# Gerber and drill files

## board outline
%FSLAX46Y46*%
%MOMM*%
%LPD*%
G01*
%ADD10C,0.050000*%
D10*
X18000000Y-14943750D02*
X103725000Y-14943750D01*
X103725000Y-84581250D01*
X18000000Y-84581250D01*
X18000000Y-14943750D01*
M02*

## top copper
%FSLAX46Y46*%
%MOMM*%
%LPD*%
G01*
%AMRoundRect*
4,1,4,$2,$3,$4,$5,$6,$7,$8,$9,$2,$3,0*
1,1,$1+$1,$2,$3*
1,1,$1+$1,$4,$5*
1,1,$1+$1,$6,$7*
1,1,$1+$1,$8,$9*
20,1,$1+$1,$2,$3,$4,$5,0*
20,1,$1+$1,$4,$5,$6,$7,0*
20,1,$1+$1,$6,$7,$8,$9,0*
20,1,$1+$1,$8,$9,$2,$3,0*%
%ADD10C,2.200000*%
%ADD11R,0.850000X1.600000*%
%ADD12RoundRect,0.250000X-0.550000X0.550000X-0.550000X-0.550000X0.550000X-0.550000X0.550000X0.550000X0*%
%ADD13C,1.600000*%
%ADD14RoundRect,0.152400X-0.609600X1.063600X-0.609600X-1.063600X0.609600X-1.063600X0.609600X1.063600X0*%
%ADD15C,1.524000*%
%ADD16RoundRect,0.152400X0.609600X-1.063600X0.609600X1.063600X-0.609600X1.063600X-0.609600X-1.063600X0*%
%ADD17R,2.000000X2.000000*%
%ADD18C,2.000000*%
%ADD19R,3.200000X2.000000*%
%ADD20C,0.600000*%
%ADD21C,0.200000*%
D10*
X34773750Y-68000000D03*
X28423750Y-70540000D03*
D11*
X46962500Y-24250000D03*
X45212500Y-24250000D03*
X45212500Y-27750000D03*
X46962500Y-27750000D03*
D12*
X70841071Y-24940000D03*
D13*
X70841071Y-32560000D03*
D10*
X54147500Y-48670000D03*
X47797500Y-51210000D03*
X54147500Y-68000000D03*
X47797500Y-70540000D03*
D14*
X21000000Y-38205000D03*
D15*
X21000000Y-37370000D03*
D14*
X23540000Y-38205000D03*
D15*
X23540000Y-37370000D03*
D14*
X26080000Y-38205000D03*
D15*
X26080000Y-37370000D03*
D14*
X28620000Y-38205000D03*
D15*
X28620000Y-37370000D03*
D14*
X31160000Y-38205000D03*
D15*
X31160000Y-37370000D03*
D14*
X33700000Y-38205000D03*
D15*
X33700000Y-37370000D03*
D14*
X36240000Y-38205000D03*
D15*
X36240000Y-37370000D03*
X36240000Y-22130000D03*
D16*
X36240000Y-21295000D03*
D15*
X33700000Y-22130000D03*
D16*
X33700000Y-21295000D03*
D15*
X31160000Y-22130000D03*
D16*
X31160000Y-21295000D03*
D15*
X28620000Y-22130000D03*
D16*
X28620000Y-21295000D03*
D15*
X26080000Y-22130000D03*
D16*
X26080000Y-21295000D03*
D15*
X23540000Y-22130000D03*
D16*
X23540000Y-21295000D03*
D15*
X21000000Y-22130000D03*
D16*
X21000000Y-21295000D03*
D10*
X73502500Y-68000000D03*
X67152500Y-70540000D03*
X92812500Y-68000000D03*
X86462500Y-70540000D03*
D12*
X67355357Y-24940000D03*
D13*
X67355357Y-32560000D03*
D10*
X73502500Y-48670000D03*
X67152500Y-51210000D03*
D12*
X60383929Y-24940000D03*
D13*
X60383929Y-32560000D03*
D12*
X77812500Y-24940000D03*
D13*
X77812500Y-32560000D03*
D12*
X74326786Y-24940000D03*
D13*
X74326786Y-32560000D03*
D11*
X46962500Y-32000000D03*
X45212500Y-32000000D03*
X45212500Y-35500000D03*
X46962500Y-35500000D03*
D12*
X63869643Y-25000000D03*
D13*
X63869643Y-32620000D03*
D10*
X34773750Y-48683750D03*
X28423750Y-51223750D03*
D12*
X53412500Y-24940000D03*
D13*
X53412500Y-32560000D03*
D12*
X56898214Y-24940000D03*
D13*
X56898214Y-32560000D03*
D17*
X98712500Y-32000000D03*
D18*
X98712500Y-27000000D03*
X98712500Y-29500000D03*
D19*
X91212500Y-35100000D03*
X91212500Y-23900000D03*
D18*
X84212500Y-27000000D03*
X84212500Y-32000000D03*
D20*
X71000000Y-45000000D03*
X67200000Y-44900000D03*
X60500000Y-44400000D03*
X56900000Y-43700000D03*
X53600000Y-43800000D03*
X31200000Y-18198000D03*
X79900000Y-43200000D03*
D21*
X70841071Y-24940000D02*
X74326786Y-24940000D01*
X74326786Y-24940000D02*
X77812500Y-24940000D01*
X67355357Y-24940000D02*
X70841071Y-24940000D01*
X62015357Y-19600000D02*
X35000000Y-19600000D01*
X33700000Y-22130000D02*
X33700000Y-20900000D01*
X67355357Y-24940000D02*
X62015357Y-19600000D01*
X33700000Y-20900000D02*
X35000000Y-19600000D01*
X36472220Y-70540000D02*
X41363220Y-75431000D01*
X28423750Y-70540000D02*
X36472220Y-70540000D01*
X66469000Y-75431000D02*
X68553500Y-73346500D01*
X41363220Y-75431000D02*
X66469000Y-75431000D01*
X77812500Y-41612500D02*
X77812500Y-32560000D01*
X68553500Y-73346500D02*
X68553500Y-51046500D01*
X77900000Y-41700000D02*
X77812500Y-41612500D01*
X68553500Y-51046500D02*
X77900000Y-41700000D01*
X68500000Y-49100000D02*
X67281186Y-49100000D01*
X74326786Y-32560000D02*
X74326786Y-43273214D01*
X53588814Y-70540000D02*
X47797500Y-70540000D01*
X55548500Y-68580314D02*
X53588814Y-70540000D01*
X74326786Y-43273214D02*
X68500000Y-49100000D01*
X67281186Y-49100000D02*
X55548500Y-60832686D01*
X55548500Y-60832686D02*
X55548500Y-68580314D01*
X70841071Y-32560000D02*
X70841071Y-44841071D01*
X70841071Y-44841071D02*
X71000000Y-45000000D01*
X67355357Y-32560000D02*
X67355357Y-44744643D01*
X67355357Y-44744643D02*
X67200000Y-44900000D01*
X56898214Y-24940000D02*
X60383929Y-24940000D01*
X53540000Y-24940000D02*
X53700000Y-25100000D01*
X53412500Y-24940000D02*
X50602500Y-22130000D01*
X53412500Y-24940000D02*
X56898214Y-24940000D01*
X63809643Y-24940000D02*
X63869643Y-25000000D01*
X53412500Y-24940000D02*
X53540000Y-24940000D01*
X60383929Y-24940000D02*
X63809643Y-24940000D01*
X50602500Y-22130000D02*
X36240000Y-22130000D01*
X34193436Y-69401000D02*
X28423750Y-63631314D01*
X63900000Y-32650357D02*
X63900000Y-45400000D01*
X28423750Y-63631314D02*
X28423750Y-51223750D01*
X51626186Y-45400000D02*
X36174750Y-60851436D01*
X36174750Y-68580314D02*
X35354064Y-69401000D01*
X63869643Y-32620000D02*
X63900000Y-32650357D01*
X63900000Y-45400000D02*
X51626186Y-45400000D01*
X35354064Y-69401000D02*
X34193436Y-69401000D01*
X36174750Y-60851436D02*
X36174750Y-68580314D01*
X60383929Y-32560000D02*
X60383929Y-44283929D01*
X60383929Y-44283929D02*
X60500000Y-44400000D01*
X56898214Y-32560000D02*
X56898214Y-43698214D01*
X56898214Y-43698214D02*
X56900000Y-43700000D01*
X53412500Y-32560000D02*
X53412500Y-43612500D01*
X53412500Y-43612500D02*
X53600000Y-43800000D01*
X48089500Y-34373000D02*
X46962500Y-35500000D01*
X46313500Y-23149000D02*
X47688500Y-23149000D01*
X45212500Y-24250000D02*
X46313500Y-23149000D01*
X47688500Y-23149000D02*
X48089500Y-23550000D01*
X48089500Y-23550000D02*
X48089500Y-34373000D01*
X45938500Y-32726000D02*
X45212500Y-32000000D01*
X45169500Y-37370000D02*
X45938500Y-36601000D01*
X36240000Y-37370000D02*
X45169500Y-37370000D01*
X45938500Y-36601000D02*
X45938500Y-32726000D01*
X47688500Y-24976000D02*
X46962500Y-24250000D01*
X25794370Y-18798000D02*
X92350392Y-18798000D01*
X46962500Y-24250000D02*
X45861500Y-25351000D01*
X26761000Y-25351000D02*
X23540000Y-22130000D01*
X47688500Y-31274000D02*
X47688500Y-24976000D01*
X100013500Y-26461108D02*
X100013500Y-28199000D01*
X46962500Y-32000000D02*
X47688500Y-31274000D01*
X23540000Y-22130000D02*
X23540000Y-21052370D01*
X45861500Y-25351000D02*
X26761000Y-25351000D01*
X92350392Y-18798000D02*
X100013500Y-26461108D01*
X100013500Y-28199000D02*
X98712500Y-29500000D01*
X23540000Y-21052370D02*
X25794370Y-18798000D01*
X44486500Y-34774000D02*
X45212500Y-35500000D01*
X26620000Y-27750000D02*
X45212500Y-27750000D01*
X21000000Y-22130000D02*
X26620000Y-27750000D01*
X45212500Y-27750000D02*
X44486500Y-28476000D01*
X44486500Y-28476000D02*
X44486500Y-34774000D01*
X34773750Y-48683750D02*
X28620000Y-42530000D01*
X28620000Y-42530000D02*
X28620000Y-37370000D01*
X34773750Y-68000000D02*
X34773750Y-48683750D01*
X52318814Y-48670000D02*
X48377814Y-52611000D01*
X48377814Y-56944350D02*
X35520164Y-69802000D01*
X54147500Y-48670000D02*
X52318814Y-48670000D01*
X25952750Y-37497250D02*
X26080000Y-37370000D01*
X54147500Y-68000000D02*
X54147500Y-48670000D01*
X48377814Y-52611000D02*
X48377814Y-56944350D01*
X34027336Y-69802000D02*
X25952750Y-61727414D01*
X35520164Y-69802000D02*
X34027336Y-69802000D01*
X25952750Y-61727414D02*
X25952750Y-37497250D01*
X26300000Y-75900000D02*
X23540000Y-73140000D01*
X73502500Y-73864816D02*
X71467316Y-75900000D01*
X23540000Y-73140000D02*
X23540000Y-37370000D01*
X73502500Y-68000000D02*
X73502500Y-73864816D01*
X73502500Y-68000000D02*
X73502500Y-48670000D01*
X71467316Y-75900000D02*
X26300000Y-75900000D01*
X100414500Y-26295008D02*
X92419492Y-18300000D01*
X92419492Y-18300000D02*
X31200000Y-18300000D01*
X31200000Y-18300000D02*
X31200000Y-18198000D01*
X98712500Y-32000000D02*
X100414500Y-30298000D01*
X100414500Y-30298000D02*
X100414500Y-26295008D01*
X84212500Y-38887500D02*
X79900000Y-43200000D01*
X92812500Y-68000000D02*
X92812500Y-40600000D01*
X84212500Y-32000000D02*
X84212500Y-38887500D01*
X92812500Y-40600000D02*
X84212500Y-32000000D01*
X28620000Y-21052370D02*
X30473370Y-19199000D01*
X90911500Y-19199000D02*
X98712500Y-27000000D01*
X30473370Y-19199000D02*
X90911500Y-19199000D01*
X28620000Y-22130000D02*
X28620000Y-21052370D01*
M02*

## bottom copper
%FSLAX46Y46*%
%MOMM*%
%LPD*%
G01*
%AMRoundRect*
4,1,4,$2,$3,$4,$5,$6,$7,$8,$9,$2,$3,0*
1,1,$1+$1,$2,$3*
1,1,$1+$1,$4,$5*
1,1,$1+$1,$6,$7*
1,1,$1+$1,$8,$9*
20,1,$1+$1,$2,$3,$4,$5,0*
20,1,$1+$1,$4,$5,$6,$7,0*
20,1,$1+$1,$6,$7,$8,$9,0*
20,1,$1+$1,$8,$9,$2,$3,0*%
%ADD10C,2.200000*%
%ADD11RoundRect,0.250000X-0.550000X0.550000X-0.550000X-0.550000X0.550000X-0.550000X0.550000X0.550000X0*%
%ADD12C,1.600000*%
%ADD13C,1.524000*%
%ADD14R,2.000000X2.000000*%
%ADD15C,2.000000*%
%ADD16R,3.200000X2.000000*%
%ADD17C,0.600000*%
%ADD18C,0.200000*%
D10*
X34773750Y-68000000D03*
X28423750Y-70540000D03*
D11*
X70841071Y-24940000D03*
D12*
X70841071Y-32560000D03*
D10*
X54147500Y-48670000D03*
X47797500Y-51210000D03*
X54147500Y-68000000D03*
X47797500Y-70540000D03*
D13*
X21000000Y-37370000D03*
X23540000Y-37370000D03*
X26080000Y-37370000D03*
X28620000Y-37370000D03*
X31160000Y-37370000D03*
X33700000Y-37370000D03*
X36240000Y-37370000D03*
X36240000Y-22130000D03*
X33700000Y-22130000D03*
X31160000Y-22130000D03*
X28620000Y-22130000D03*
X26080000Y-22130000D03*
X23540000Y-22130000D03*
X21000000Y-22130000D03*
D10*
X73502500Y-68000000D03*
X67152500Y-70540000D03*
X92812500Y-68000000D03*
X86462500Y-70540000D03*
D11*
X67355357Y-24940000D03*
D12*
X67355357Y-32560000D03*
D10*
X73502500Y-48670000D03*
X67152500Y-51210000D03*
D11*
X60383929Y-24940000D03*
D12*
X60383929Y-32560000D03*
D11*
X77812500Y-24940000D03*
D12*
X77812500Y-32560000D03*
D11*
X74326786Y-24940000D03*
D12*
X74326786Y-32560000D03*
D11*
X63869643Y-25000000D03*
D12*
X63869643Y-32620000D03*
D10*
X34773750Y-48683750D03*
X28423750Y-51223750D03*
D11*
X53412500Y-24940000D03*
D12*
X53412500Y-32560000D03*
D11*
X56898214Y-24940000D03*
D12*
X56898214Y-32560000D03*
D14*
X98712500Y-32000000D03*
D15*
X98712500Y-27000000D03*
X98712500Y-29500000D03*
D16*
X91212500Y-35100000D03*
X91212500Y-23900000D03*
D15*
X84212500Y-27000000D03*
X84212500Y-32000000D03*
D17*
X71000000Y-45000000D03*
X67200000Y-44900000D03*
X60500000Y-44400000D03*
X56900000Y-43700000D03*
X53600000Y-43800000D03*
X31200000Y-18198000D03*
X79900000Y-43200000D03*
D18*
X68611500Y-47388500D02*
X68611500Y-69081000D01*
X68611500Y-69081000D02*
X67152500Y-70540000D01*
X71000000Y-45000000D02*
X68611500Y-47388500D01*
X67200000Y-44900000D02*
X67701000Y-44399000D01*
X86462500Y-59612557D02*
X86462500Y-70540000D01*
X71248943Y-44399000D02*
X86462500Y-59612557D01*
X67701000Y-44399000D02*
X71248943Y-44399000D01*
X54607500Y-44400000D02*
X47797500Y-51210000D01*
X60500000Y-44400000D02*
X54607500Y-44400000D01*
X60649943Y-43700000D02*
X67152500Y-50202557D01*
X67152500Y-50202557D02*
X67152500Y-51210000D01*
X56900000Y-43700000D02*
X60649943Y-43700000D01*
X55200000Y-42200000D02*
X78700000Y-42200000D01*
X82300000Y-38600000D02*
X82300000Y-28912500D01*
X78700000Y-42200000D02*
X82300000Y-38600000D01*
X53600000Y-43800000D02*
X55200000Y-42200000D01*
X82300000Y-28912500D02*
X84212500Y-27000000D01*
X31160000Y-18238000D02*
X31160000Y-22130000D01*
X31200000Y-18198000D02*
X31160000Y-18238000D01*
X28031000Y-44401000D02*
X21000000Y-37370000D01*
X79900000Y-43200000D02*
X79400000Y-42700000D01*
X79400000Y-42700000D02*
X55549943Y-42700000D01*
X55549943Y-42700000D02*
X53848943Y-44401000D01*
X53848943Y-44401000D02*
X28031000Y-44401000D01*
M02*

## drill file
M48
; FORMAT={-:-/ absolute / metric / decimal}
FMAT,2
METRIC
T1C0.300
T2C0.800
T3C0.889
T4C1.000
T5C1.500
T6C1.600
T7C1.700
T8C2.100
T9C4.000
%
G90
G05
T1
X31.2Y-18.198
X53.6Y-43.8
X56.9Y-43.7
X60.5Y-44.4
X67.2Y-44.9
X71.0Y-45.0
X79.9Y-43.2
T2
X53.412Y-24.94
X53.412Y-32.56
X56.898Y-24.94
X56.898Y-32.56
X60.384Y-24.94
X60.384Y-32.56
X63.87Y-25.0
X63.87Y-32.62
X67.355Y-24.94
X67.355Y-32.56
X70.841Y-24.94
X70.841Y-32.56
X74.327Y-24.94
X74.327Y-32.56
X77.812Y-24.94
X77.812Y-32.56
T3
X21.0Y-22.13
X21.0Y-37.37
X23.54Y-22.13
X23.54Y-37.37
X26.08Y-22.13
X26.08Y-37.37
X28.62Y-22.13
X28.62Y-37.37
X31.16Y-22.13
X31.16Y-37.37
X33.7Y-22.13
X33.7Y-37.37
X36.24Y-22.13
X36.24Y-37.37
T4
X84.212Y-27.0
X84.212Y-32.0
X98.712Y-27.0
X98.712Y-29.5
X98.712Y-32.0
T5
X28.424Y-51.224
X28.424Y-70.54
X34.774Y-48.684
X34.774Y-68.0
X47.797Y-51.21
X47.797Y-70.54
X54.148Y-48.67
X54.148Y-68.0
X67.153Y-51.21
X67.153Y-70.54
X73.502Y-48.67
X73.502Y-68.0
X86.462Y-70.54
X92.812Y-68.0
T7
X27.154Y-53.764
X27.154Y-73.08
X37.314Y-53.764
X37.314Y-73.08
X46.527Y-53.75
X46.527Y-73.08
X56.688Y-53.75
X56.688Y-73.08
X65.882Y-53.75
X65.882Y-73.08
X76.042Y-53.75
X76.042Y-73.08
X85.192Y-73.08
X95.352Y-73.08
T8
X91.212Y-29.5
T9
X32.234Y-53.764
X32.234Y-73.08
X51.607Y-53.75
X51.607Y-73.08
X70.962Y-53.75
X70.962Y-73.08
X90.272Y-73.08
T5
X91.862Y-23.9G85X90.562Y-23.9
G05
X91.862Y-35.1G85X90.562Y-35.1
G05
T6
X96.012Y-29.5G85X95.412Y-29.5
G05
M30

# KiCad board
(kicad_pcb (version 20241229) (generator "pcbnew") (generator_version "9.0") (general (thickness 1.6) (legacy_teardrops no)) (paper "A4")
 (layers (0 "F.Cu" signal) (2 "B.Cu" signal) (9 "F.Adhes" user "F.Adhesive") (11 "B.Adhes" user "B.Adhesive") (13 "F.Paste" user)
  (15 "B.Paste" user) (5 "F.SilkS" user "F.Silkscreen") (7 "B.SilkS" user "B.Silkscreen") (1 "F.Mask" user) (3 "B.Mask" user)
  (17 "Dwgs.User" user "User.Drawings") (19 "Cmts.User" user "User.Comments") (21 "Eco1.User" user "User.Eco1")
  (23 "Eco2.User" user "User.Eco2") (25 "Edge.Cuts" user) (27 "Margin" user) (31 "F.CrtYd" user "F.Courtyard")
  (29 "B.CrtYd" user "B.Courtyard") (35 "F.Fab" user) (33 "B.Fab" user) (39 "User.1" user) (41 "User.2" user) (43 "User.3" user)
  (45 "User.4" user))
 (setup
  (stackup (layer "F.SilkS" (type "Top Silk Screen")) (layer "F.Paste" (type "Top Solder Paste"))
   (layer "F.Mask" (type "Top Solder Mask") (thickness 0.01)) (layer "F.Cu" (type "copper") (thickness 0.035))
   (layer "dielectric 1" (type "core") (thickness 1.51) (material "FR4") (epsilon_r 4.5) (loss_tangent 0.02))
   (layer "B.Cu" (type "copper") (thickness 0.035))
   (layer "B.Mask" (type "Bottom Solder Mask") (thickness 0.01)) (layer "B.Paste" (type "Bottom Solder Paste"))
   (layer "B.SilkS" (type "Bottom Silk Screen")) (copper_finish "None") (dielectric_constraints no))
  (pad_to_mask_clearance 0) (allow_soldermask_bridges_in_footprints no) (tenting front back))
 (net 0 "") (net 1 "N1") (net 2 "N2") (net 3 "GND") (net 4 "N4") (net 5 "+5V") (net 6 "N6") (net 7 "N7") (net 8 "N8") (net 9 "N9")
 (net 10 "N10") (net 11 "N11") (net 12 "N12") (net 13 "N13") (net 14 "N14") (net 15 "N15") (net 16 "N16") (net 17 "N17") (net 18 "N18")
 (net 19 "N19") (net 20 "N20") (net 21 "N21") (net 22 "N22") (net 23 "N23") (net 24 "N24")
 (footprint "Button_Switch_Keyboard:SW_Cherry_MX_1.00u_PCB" (layer "F.Cu") (at 34.77375 68)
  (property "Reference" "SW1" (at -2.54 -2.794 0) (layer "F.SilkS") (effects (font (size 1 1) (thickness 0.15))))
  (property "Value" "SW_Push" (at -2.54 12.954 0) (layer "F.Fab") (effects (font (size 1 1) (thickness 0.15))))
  (pad "" np_thru_hole circle (at -7.62 5.08) (size 1.7 1.7) (drill 1.7) (layers "*.Cu" "*.Mask"))
  (pad "" np_thru_hole circle (at -2.54 5.08) (size 4 4) (drill 4) (layers "*.Cu" "*.Mask"))
  (pad "" np_thru_hole circle (at 2.54 5.08) (size 1.7 1.7) (drill 1.7) (layers "*.Cu" "*.Mask"))
  (pad "1" thru_hole circle (at 0 0) (size 2.2 2.2) (drill 1.5) (layers "*.Cu" "*.Mask") (remove_unused_layers no) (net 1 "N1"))
  (pad "2" thru_hole circle (at -6.35 2.54) (size 2.2 2.2) (drill 1.5) (layers "*.Cu" "*.Mask") (remove_unused_layers no) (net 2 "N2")))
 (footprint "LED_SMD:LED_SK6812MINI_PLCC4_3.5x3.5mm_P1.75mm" (layer "F.Cu") (at 46.0875 26 -90)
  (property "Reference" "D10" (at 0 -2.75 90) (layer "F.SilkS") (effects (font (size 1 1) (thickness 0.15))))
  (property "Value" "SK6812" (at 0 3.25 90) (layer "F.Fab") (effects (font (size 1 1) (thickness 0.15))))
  (pad "1" smd rect (at -1.75 -0.875 270) (size 1.6 0.85) (layers "F.Cu" "F.Mask" "F.Paste") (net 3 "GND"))
  (pad "2" smd rect (at -1.75 0.875 270) (size 1.6 0.85) (layers "F.Cu" "F.Mask" "F.Paste") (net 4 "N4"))
  (pad "3" smd rect (at 1.75 0.875 270) (size 1.6 0.85) (layers "F.Cu" "F.Mask" "F.Paste") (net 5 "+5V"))
  (pad "4" smd rect (at 1.75 -0.875 270) (size 1.6 0.85) (layers "F.Cu" "F.Mask" "F.Paste") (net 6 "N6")))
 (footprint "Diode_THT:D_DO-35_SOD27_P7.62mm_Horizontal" (layer "F.Cu") (at 70.841071 24.94 -90)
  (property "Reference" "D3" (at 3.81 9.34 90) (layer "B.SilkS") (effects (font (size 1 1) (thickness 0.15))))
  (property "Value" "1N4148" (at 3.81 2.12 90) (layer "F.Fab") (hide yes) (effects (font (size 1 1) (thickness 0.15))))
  (pad "1" thru_hole roundrect (at 0 0 270) (size 1.6 1.6) (drill 0.8) (layers "*.Cu" "*.Mask") (remove_unused_layers no)
   (roundrect_rratio 0.15625) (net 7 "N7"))
  (pad "2" thru_hole circle (at 7.62 0 270) (size 1.6 1.6) (drill 0.8) (layers "*.Cu" "*.Mask") (remove_unused_layers no) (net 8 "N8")))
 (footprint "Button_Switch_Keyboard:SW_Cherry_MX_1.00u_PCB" (layer "F.Cu") (at 54.1475 48.67)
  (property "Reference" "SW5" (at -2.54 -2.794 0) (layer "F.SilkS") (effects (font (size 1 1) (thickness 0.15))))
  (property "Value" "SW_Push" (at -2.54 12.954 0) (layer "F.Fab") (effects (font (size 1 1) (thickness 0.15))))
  (pad "" np_thru_hole circle (at -7.62 5.08) (size 1.7 1.7) (drill 1.7) (layers "*.Cu" "*.Mask"))
  (pad "" np_thru_hole circle (at -2.54 5.08) (size 4 4) (drill 4) (layers "*.Cu" "*.Mask"))
  (pad "" np_thru_hole circle (at 2.54 5.08) (size 1.7 1.7) (drill 1.7) (layers "*.Cu" "*.Mask"))
  (pad "1" thru_hole circle (at 0 0) (size 2.2 2.2) (drill 1.5) (layers "*.Cu" "*.Mask") (remove_unused_layers no) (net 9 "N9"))
  (pad "2" thru_hole circle (at -6.35 2.54) (size 2.2 2.2) (drill 1.5) (layers "*.Cu" "*.Mask") (remove_unused_layers no) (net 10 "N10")))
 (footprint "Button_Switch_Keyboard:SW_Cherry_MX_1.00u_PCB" (layer "F.Cu") (at 54.1475 68)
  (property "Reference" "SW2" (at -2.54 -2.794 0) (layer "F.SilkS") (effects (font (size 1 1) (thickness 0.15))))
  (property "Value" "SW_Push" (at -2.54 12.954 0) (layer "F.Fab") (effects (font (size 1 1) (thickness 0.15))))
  (pad "" np_thru_hole circle (at -7.62 5.08) (size 1.7 1.7) (drill 1.7) (layers "*.Cu" "*.Mask"))
  (pad "" np_thru_hole circle (at -2.54 5.08) (size 4 4) (drill 4) (layers "*.Cu" "*.Mask"))
  (pad "" np_thru_hole circle (at 2.54 5.08) (size 1.7 1.7) (drill 1.7) (layers "*.Cu" "*.Mask"))
  (pad "1" thru_hole circle (at 0 0) (size 2.2 2.2) (drill 1.5) (layers "*.Cu" "*.Mask") (remove_unused_layers no) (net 9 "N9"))
  (pad "2" thru_hole circle (at -6.35 2.54) (size 2.2 2.2) (drill 1.5) (layers "*.Cu" "*.Mask") (remove_unused_layers no) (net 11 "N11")))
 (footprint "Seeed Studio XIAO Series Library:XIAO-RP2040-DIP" (layer "F.Cu") (at 28.62 29.75 90)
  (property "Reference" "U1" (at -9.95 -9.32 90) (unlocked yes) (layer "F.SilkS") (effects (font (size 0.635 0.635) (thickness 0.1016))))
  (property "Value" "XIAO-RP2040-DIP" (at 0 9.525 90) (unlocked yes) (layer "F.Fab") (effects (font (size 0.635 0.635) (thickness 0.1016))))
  (pad "1" smd roundrect (at -8.455 -7.62 270) (size 2.432 1.524) (layers "F.Cu" "F.Mask") (roundrect_rratio 0.1) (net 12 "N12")
   (thermal_bridge_angle 45))
  (pad "1" thru_hole circle (at -7.62 -7.62 270) (size 1.524 1.524) (drill 0.889) (layers "*.Cu" "*.Mask") (remove_unused_layers no)
   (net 12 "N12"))
  (pad "2" smd roundrect (at -8.455 -5.08 270) (size 2.432 1.524) (layers "F.Cu" "F.Mask") (roundrect_rratio 0.1) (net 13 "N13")
   (thermal_bridge_angle 45))
  (pad "2" thru_hole circle (at -7.62 -5.08 270) (size 1.524 1.524) (drill 0.889) (layers "*.Cu" "*.Mask") (remove_unused_layers no)
   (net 13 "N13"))
  (pad "3" smd roundrect (at -8.455 -2.54 270) (size 2.432 1.524) (layers "F.Cu" "F.Mask") (roundrect_rratio 0.1) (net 9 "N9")
   (thermal_bridge_angle 45))
  (pad "3" thru_hole circle (at -7.62 -2.54 270) (size 1.524 1.524) (drill 0.889) (layers "*.Cu" "*.Mask") (remove_unused_layers no)
   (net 9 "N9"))
  (pad "4" smd roundrect (at -8.455 0 270) (size 2.432 1.524) (layers "F.Cu" "F.Mask") (roundrect_rratio 0.1) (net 1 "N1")
   (thermal_bridge_angle 45))
  (pad "4" thru_hole circle (at -7.62 0 270) (size 1.524 1.524) (drill 0.889) (layers "*.Cu" "*.Mask") (remove_unused_layers no)
   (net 1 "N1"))
  (pad "5" smd roundrect (at -8.455 2.54 270) (size 2.432 1.524) (layers "F.Cu" "F.Mask") (roundrect_rratio 0.1) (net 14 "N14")
   (thermal_bridge_angle 45))
  (pad "5" thru_hole circle (at -7.62 2.54 270) (size 1.524 1.524) (drill 0.889) (layers "*.Cu" "*.Mask") (remove_unused_layers no)
   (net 14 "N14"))
  (pad "6" smd roundrect (at -8.455 5.08 270) (size 2.432 1.524) (layers "F.Cu" "F.Mask") (roundrect_rratio 0.1) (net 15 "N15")
   (thermal_bridge_angle 45))
  (pad "6" thru_hole circle (at -7.62 5.08 270) (size 1.524 1.524) (drill 0.889) (layers "*.Cu" "*.Mask") (remove_unused_layers no)
   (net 15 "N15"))
  (pad "7" smd roundrect (at -8.455 7.62 270) (size 2.432 1.524) (layers "F.Cu" "F.Mask") (roundrect_rratio 0.1) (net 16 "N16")
   (thermal_bridge_angle 45))
  (pad "7" thru_hole circle (at -7.62 7.62 270) (size 1.524 1.524) (drill 0.889) (layers "*.Cu" "*.Mask") (remove_unused_layers no)
   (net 16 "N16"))
  (pad "8" thru_hole circle (at 7.62 7.62 90) (size 1.524 1.524) (drill 0.889) (layers "*.Cu" "*.Mask") (remove_unused_layers no)
   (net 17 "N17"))
  (pad "8" smd roundrect (at 8.455 7.62 90) (size 2.432 1.524) (layers "F.Cu" "F.Mask") (roundrect_rratio 0.1) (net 17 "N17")
   (thermal_bridge_angle 45))
  (pad "9" thru_hole circle (at 7.62 5.08 90) (size 1.524 1.524) (drill 0.889) (layers "*.Cu" "*.Mask") (remove_unused_layers no)
   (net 7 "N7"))
  (pad "9" smd roundrect (at 8.455 5.08 90) (size 2.432 1.524) (layers "F.Cu" "F.Mask") (roundrect_rratio 0.1) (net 7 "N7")
   (thermal_bridge_angle 45))
  (pad "10" thru_hole circle (at 7.62 2.54 90) (size 1.524 1.524) (drill 0.889) (layers "*.Cu" "*.Mask") (remove_unused_layers no)
   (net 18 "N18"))
  (pad "10" smd roundrect (at 8.455 2.54 90) (size 2.432 1.524) (layers "F.Cu" "F.Mask") (roundrect_rratio 0.1) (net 18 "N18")
   (thermal_bridge_angle 45))
  (pad "11" thru_hole circle (at 7.62 0 90) (size 1.524 1.524) (drill 0.889) (layers "*.Cu" "*.Mask") (remove_unused_layers no)
   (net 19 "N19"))
  (pad "11" smd roundrect (at 8.455 0 90) (size 2.432 1.524) (layers "F.Cu" "F.Mask") (roundrect_rratio 0.1) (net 19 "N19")
   (thermal_bridge_angle 45))
  (pad "12" thru_hole circle (at 7.62 -2.54 90) (size 1.524 1.524) (drill 0.889) (layers "*.Cu" "*.Mask") (remove_unused_layers no)
   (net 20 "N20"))
  (pad "12" smd roundrect (at 8.455 -2.54 90) (size 2.432 1.524) (layers "F.Cu" "F.Mask") (roundrect_rratio 0.1) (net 20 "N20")
   (thermal_bridge_angle 45))
  (pad "13" thru_hole circle (at 7.62 -5.08 90) (size 1.524 1.524) (drill 0.889) (layers "*.Cu" "*.Mask") (remove_unused_layers no)
   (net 3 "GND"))
  (pad "13" smd roundrect (at 8.455 -5.08 90) (size 2.432 1.524) (layers "F.Cu" "F.Mask") (roundrect_rratio 0.1) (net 3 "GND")
   (thermal_bridge_angle 45))
  (pad "14" thru_hole circle (at 7.62 -7.62 90) (size 1.524 1.524) (drill 0.889) (layers "*.Cu" "*.Mask") (remove_unused_layers no)
   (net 5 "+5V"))
  (pad "14" smd roundrect (at 8.455 -7.62 90) (size 2.432 1.524) (layers "F.Cu" "F.Mask") (roundrect_rratio 0.1) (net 5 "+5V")
   (thermal_bridge_angle 45)))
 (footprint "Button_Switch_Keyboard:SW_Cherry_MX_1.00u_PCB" (layer "F.Cu") (at 73.5025 68)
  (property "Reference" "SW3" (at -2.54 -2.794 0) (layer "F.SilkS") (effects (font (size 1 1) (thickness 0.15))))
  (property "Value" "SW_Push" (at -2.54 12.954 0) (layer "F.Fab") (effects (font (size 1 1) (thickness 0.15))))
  (pad "" np_thru_hole circle (at -7.62 5.08) (size 1.7 1.7) (drill 1.7) (layers "*.Cu" "*.Mask"))
  (pad "" np_thru_hole circle (at -2.54 5.08) (size 4 4) (drill 4) (layers "*.Cu" "*.Mask"))
  (pad "" np_thru_hole circle (at 2.54 5.08) (size 1.7 1.7) (drill 1.7) (layers "*.Cu" "*.Mask"))
  (pad "1" thru_hole circle (at 0 0) (size 2.2 2.2) (drill 1.5) (layers "*.Cu" "*.Mask") (remove_unused_layers no) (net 13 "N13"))
  (pad "2" thru_hole circle (at -6.35 2.54) (size 2.2 2.2) (drill 1.5) (layers "*.Cu" "*.Mask") (remove_unused_layers no) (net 8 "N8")))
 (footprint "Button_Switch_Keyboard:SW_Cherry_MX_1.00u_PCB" (layer "F.Cu") (at 92.8125 68)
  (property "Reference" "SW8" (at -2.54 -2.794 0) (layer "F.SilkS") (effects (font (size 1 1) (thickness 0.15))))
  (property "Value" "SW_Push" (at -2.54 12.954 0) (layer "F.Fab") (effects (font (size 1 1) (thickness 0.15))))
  (pad "" np_thru_hole circle (at -7.62 5.08) (size 1.7 1.7) (drill 1.7) (layers "*.Cu" "*.Mask"))
  (pad "" np_thru_hole circle (at -2.54 5.08) (size 4 4) (drill 4) (layers "*.Cu" "*.Mask"))
  (pad "" np_thru_hole circle (at 2.54 5.08) (size 1.7 1.7) (drill 1.7) (layers "*.Cu" "*.Mask"))
  (pad "1" thru_hole circle (at 0 0) (size 2.2 2.2) (drill 1.5) (layers "*.Cu" "*.Mask") (remove_unused_layers no) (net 12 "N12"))
  (pad "2" thru_hole circle (at -6.35 2.54) (size 2.2 2.2) (drill 1.5) (layers "*.Cu" "*.Mask") (remove_unused_layers no) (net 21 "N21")))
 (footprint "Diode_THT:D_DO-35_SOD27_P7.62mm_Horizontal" (layer "F.Cu") (at 67.355357 24.94 -90)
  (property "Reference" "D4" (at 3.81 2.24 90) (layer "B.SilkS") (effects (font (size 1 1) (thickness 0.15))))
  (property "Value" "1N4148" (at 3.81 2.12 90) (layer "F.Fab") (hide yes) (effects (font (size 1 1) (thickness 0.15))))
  (pad "1" thru_hole roundrect (at 0 0 270) (size 1.6 1.6) (drill 0.8) (layers "*.Cu" "*.Mask") (remove_unused_layers no)
   (roundrect_rratio 0.15625) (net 7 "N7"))
  (pad "2" thru_hole circle (at 7.62 0 270) (size 1.6 1.6) (drill 0.8) (layers "*.Cu" "*.Mask") (remove_unused_layers no) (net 21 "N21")))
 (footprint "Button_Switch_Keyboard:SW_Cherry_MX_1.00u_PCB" (layer "F.Cu") (at 73.5025 48.67)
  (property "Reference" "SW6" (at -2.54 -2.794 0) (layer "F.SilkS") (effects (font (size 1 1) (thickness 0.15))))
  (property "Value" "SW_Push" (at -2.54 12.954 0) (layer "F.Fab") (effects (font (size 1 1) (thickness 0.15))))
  (pad "" np_thru_hole circle (at -7.62 5.08) (size 1.7 1.7) (drill 1.7) (layers "*.Cu" "*.Mask"))
  (pad "" np_thru_hole circle (at -2.54 5.08) (size 4 4) (drill 4) (layers "*.Cu" "*.Mask"))
  (pad "" np_thru_hole circle (at 2.54 5.08) (size 1.7 1.7) (drill 1.7) (layers "*.Cu" "*.Mask"))
  (pad "1" thru_hole circle (at 0 0) (size 2.2 2.2) (drill 1.5) (layers "*.Cu" "*.Mask") (remove_unused_layers no) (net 13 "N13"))
  (pad "2" thru_hole circle (at -6.35 2.54) (size 2.2 2.2) (drill 1.5) (layers "*.Cu" "*.Mask") (remove_unused_layers no) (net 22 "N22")))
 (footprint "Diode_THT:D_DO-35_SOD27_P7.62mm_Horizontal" (layer "F.Cu") (at 60.383929 24.94 -90)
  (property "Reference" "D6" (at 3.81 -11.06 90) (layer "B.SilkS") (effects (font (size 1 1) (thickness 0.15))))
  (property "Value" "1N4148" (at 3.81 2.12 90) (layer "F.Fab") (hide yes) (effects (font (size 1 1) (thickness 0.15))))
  (pad "1" thru_hole roundrect (at 0 0 270) (size 1.6 1.6) (drill 0.8) (layers "*.Cu" "*.Mask") (remove_unused_layers no)
   (roundrect_rratio 0.15625) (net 17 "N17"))
  (pad "2" thru_hole circle (at 7.62 0 270) (size 1.6 1.6) (drill 0.8) (layers "*.Cu" "*.Mask") (remove_unused_layers no) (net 10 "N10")))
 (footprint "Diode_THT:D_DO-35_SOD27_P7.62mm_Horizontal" (layer "F.Cu") (at 77.8125 24.94 -90)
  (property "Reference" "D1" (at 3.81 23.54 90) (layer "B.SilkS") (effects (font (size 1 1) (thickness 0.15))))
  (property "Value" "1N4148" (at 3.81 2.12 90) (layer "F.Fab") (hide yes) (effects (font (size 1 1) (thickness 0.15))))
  (pad "1" thru_hole roundrect (at 0 0 270) (size 1.6 1.6) (drill 0.8) (layers "*.Cu" "*.Mask") (remove_unused_layers no)
   (roundrect_rratio 0.15625) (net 7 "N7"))
  (pad "2" thru_hole circle (at 7.62 0 270) (size 1.6 1.6) (drill 0.8) (layers "*.Cu" "*.Mask") (remove_unused_layers no) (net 2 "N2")))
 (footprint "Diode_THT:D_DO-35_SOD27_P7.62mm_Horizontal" (layer "F.Cu") (at 74.326786 24.94 -90)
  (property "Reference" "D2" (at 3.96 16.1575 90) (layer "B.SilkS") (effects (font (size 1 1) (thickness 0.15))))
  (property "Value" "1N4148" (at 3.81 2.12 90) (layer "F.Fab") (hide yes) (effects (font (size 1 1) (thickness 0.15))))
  (pad "1" thru_hole roundrect (at 0 0 270) (size 1.6 1.6) (drill 0.8) (layers "*.Cu" "*.Mask") (remove_unused_layers no)
   (roundrect_rratio 0.15625) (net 7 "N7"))
  (pad "2" thru_hole circle (at 7.62 0 270) (size 1.6 1.6) (drill 0.8) (layers "*.Cu" "*.Mask") (remove_unused_layers no) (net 11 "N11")))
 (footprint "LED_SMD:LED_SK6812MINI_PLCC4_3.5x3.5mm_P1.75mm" (layer "F.Cu") (at 46.0875 33.75 -90)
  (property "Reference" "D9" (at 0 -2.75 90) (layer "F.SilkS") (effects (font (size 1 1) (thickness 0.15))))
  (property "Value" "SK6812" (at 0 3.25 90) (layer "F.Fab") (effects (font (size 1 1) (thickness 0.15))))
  (pad "1" smd rect (at -1.75 -0.875 270) (size 1.6 0.85) (layers "F.Cu" "F.Mask" "F.Paste") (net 3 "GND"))
  (pad "2" smd rect (at -1.75 0.875 270) (size 1.6 0.85) (layers "F.Cu" "F.Mask" "F.Paste") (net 16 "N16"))
  (pad "3" smd rect (at 1.75 0.875 270) (size 1.6 0.85) (layers "F.Cu" "F.Mask" "F.Paste") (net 5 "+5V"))
  (pad "4" smd rect (at 1.75 -0.875 270) (size 1.6 0.85) (layers "F.Cu" "F.Mask" "F.Paste") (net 4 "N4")))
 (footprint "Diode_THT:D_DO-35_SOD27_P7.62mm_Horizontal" (layer "F.Cu") (at 63.869643 25 -90)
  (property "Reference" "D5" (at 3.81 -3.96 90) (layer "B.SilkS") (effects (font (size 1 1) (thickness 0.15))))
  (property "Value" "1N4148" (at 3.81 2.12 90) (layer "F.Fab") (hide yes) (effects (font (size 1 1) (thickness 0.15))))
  (pad "1" thru_hole roundrect (at 0 0 270) (size 1.6 1.6) (drill 0.8) (layers "*.Cu" "*.Mask") (remove_unused_layers no)
   (roundrect_rratio 0.15625) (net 17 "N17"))
  (pad "2" thru_hole circle (at 7.62 0 270) (size 1.6 1.6) (drill 0.8) (layers "*.Cu" "*.Mask") (remove_unused_layers no) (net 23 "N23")))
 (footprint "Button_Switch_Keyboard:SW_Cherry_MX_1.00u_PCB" (layer "F.Cu") (at 34.77375 48.68375)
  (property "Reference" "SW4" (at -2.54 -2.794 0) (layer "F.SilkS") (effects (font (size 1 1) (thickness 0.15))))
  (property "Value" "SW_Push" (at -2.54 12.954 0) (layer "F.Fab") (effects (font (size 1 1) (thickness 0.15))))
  (pad "" np_thru_hole circle (at -7.62 5.08) (size 1.7 1.7) (drill 1.7) (layers "*.Cu" "*.Mask"))
  (pad "" np_thru_hole circle (at -2.54 5.08) (size 4 4) (drill 4) (layers "*.Cu" "*.Mask"))
  (pad "" np_thru_hole circle (at 2.54 5.08) (size 1.7 1.7) (drill 1.7) (layers "*.Cu" "*.Mask"))
  (pad "1" thru_hole circle (at 0 0) (size 2.2 2.2) (drill 1.5) (layers "*.Cu" "*.Mask") (remove_unused_layers no) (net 1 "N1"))
  (pad "2" thru_hole circle (at -6.35 2.54) (size 2.2 2.2) (drill 1.5) (layers "*.Cu" "*.Mask") (remove_unused_layers no) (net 23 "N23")))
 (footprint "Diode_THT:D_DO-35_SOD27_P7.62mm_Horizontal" (layer "F.Cu") (at 53.4125 24.94 -90)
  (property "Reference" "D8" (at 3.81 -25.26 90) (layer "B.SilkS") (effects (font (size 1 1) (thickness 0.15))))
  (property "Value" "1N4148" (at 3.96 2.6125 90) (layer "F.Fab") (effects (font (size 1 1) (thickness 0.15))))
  (pad "1" thru_hole roundrect (at 0 0 270) (size 1.6 1.6) (drill 0.8) (layers "*.Cu" "*.Mask") (remove_unused_layers no)
   (roundrect_rratio 0.15625) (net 17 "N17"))
  (pad "2" thru_hole circle (at 7.62 0 270) (size 1.6 1.6) (drill 0.8) (layers "*.Cu" "*.Mask") (remove_unused_layers no) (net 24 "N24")))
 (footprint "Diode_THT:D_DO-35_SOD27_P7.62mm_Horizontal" (layer "F.Cu") (at 56.898214 24.94 -90)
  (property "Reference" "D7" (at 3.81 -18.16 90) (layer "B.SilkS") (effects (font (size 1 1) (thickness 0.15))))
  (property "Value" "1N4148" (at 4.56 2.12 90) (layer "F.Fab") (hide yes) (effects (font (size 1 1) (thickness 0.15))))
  (pad "1" thru_hole roundrect (at 0 0 270) (size 1.6 1.6) (drill 0.8) (layers "*.Cu" "*.Mask") (remove_unused_layers no)
   (roundrect_rratio 0.15625) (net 17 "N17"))
  (pad "2" thru_hole circle (at 7.62 0 270) (size 1.6 1.6) (drill 0.8) (layers "*.Cu" "*.Mask") (remove_unused_layers no) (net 22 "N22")))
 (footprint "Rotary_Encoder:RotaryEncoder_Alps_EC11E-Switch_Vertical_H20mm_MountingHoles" (layer "F.Cu") (at 98.7125 32 180)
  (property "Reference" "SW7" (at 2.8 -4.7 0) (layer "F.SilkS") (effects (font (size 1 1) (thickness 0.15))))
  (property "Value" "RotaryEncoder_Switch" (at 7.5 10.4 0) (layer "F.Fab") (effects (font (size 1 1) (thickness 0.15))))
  (pad "" np_thru_hole oval (at 3 2.5 180) (size 2.2 1.6) (drill oval 2.2 1.6) (layers "*.Mask"))
  (pad "" np_thru_hole circle (at 7.5 2.5 180) (size 2.1 2.1) (drill 2.1) (layers "*.Mask"))
  (pad "A" thru_hole rect (at 0 0 180) (size 2 2) (drill 1) (layers "*.Cu" "*.Mask") (remove_unused_layers no) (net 18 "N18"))
  (pad "B" thru_hole circle (at 0 5 180) (size 2 2) (drill 1) (layers "*.Cu" "*.Mask") (remove_unused_layers no) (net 19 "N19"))
  (pad "C" thru_hole circle (at 0 2.5 180) (size 2 2) (drill 1) (layers "*.Cu" "*.Mask") (remove_unused_layers no) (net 3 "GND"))
  (pad "MP" thru_hole rect (at 7.5 -3.1 180) (size 3.2 2) (drill oval 2.8 1.5) (layers "*.Cu" "*.Mask") (remove_unused_layers no))
  (pad "MP" thru_hole rect (at 7.5 8.1 180) (size 3.2 2) (drill oval 2.8 1.5) (layers "*.Cu" "*.Mask") (remove_unused_layers no))
  (pad "S1" thru_hole circle (at 14.5 5 180) (size 2 2) (drill 1) (layers "*.Cu" "*.Mask") (remove_unused_layers no) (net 24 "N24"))
  (pad "S2" thru_hole circle (at 14.5 0 180) (size 2 2) (drill 1) (layers "*.Cu" "*.Mask") (remove_unused_layers no) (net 12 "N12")))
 (gr_rect (start 18 14.94375) (end 103.725 84.58125) (stroke (width 0.05) (type default)) (fill no) (layer "Edge.Cuts"))
 (segment (start 70.841071 24.94) (end 74.326786 24.94) (width 0.2) (layer "F.Cu") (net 7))
 (segment (start 74.326786 24.94) (end 77.8125 24.94) (width 0.2) (layer "F.Cu") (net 7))
 (segment (start 67.355357 24.94) (end 70.841071 24.94) (width 0.2) (layer "F.Cu") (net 7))
 (segment (start 62.015357 19.6) (end 35 19.6) (width 0.2) (layer "F.Cu") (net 7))
 (segment (start 33.7 22.13) (end 33.7 20.9) (width 0.2) (layer "F.Cu") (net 7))
 (segment (start 67.355357 24.94) (end 62.015357 19.6) (width 0.2) (layer "F.Cu") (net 7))
 (segment (start 33.7 20.9) (end 35 19.6) (width 0.2) (layer "F.Cu") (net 7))
 (segment (start 36.47222 70.54) (end 41.36322 75.431) (width 0.2) (layer "F.Cu") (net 2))
 (segment (start 28.42375 70.54) (end 36.47222 70.54) (width 0.2) (layer "F.Cu") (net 2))
 (segment (start 66.469 75.431) (end 68.5535 73.3465) (width 0.2) (layer "F.Cu") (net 2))
 (segment (start 41.36322 75.431) (end 66.469 75.431) (width 0.2) (layer "F.Cu") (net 2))
 (segment (start 77.8125 41.6125) (end 77.8125 32.56) (width 0.2) (layer "F.Cu") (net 2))
 (segment (start 68.5535 73.3465) (end 68.5535 51.0465) (width 0.2) (layer "F.Cu") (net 2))
 (segment (start 77.9 41.7) (end 77.8125 41.6125) (width 0.2) (layer "F.Cu") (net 2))
 (segment (start 68.5535 51.0465) (end 77.9 41.7) (width 0.2) (layer "F.Cu") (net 2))
 (segment (start 68.5 49.1) (end 67.281186 49.1) (width 0.2) (layer "F.Cu") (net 11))
 (segment (start 74.326786 32.56) (end 74.326786 43.273214) (width 0.2) (layer "F.Cu") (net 11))
 (segment (start 53.588814 70.54) (end 47.7975 70.54) (width 0.2) (layer "F.Cu") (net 11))
 (segment (start 55.5485 68.580314) (end 53.588814 70.54) (width 0.2) (layer "F.Cu") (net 11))
 (segment (start 74.326786 43.273214) (end 68.5 49.1) (width 0.2) (layer "F.Cu") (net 11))
 (segment (start 67.281186 49.1) (end 55.5485 60.832686) (width 0.2) (layer "F.Cu") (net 11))
 (segment (start 55.5485 60.832686) (end 55.5485 68.580314) (width 0.2) (layer "F.Cu") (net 11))
 (segment (start 70.841071 32.56) (end 70.841071 44.841071) (width 0.2) (layer "F.Cu") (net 8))
 (segment (start 70.841071 44.841071) (end 71 45) (width 0.2) (layer "F.Cu") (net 8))
 (via (at 71 45) (size 0.6) (drill 0.3) (layers "F.Cu" "B.Cu") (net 8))
 (segment (start 68.6115 47.3885) (end 68.6115 69.081) (width 0.2) (layer "B.Cu") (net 8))
 (segment (start 68.6115 69.081) (end 67.1525 70.54) (width 0.2) (layer "B.Cu") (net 8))
 (segment (start 71 45) (end 68.6115 47.3885) (width 0.2) (layer "B.Cu") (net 8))
 (segment (start 67.355357 32.56) (end 67.355357 44.744643) (width 0.2) (layer "F.Cu") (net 21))
 (segment (start 67.355357 44.744643) (end 67.2 44.9) (width 0.2) (layer "F.Cu") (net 21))
 (via (at 67.2 44.9) (size 0.6) (drill 0.3) (layers "F.Cu" "B.Cu") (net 21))
 (segment (start 67.2 44.9) (end 67.701 44.399) (width 0.2) (layer "B.Cu") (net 21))
 (segment (start 86.4625 59.612557) (end 86.4625 70.54) (width 0.2) (layer "B.Cu") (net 21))
 (segment (start 71.248943 44.399) (end 86.4625 59.612557) (width 0.2) (layer "B.Cu") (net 21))
 (segment (start 67.701 44.399) (end 71.248943 44.399) (width 0.2) (layer "B.Cu") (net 21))
 (segment (start 56.898214 24.94) (end 60.383929 24.94) (width 0.2) (layer "F.Cu") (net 17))
 (segment (start 53.54 24.94) (end 53.7 25.1) (width 0.2) (layer "F.Cu") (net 17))
 (segment (start 53.4125 24.94) (end 50.6025 22.13) (width 0.2) (layer "F.Cu") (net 17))
 (segment (start 53.4125 24.94) (end 56.898214 24.94) (width 0.2) (layer "F.Cu") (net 17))
 (segment (start 63.809643 24.94) (end 63.869643 25) (width 0.2) (layer "F.Cu") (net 17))
 (segment (start 53.4125 24.94) (end 53.54 24.94) (width 0.2) (layer "F.Cu") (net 17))
 (segment (start 60.383929 24.94) (end 63.809643 24.94) (width 0.2) (layer "F.Cu") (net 17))
 (segment (start 50.6025 22.13) (end 36.24 22.13) (width 0.2) (layer "F.Cu") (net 17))
 (segment (start 34.193436 69.401) (end 28.42375 63.631314) (width 0.2) (layer "F.Cu") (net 23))
 (segment (start 63.9 32.650357) (end 63.9 45.4) (width 0.2) (layer "F.Cu") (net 23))
 (segment (start 28.42375 63.631314) (end 28.42375 51.22375) (width 0.2) (layer "F.Cu") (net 23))
 (segment (start 51.626186 45.4) (end 36.17475 60.851436) (width 0.2) (layer "F.Cu") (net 23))
 (segment (start 36.17475 68.580314) (end 35.354064 69.401) (width 0.2) (layer "F.Cu") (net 23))
 (segment (start 63.869643 32.62) (end 63.9 32.650357) (width 0.2) (layer "F.Cu") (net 23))
 (segment (start 63.9 45.4) (end 51.626186 45.4) (width 0.2) (layer "F.Cu") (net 23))
 (segment (start 35.354064 69.401) (end 34.193436 69.401) (width 0.2) (layer "F.Cu") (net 23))
 (segment (start 36.17475 60.851436) (end 36.17475 68.580314) (width 0.2) (layer "F.Cu") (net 23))
 (segment (start 60.383929 32.56) (end 60.383929 44.283929) (width 0.2) (layer "F.Cu") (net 10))
 (segment (start 60.383929 44.283929) (end 60.5 44.4) (width 0.2) (layer "F.Cu") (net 10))
 (via (at 60.5 44.4) (size 0.6) (drill 0.3) (layers "F.Cu" "B.Cu") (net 10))
 (segment (start 54.6075 44.4) (end 47.7975 51.21) (width 0.2) (layer "B.Cu") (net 10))
 (segment (start 60.5 44.4) (end 54.6075 44.4) (width 0.2) (layer "B.Cu") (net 10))
 (segment (start 56.898214 32.56) (end 56.898214 43.698214) (width 0.2) (layer "F.Cu") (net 22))
 (segment (start 56.898214 43.698214) (end 56.9 43.7) (width 0.2) (layer "F.Cu") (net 22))
 (via (at 56.9 43.7) (size 0.6) (drill 0.3) (layers "F.Cu" "B.Cu") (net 22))
 (segment (start 60.649943 43.7) (end 67.1525 50.202557) (width 0.2) (layer "B.Cu") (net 22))
 (segment (start 67.1525 50.202557) (end 67.1525 51.21) (width 0.2) (layer "B.Cu") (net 22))
 (segment (start 56.9 43.7) (end 60.649943 43.7) (width 0.2) (layer "B.Cu") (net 22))
 (segment (start 53.4125 32.56) (end 53.4125 43.6125) (width 0.2) (layer "F.Cu") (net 24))
 (segment (start 53.4125 43.6125) (end 53.6 43.8) (width 0.2) (layer "F.Cu") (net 24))
 (via (at 53.6 43.8) (size 0.6) (drill 0.3) (layers "F.Cu" "B.Cu") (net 24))
 (segment (start 55.2 42.2) (end 78.7 42.2) (width 0.2) (layer "B.Cu") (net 24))
 (segment (start 82.3 38.6) (end 82.3 28.9125) (width 0.2) (layer "B.Cu") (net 24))
 (segment (start 78.7 42.2) (end 82.3 38.6) (width 0.2) (layer "B.Cu") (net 24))
 (segment (start 53.6 43.8) (end 55.2 42.2) (width 0.2) (layer "B.Cu") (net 24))
 (segment (start 82.3 28.9125) (end 84.2125 27) (width 0.2) (layer "B.Cu") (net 24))
 (segment (start 48.0895 34.373) (end 46.9625 35.5) (width 0.2) (layer "F.Cu") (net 4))
 (segment (start 46.3135 23.149) (end 47.6885 23.149) (width 0.2) (layer "F.Cu") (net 4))
 (segment (start 45.2125 24.25) (end 46.3135 23.149) (width 0.2) (layer "F.Cu") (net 4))
 (segment (start 47.6885 23.149) (end 48.0895 23.55) (width 0.2) (layer "F.Cu") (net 4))
 (segment (start 48.0895 23.55) (end 48.0895 34.373) (width 0.2) (layer "F.Cu") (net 4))
 (segment (start 45.9385 32.726) (end 45.2125 32) (width 0.2) (layer "F.Cu") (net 16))
 (segment (start 45.1695 37.37) (end 45.9385 36.601) (width 0.2) (layer "F.Cu") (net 16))
 (segment (start 36.24 37.37) (end 45.1695 37.37) (width 0.2) (layer "F.Cu") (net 16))
 (segment (start 45.9385 36.601) (end 45.9385 32.726) (width 0.2) (layer "F.Cu") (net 16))
 (segment (start 47.6885 24.976) (end 46.9625 24.25) (width 0.2) (layer "F.Cu") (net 3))
 (segment (start 25.79437 18.798) (end 92.350392 18.798) (width 0.2) (layer "F.Cu") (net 3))
 (segment (start 46.9625 24.25) (end 45.8615 25.351) (width 0.2) (layer "F.Cu") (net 3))
 (segment (start 26.761 25.351) (end 23.54 22.13) (width 0.2) (layer "F.Cu") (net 3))
 (segment (start 47.6885 31.274) (end 47.6885 24.976) (width 0.2) (layer "F.Cu") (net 3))
 (segment (start 100.0135 26.461108) (end 100.0135 28.199) (width 0.2) (layer "F.Cu") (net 3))
 (segment (start 46.9625 32) (end 47.6885 31.274) (width 0.2) (layer "F.Cu") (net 3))
 (segment (start 23.54 22.13) (end 23.54 21.05237) (width 0.2) (layer "F.Cu") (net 3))
 (segment (start 45.8615 25.351) (end 26.761 25.351) (width 0.2) (layer "F.Cu") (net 3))
 (segment (start 92.350392 18.798) (end 100.0135 26.461108) (width 0.2) (layer "F.Cu") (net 3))
 (segment (start 100.0135 28.199) (end 98.7125 29.5) (width 0.2) (layer "F.Cu") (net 3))
 (segment (start 23.54 21.05237) (end 25.79437 18.798) (width 0.2) (layer "F.Cu") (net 3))
 (segment (start 44.4865 34.774) (end 45.2125 35.5) (width 0.2) (layer "F.Cu") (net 5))
 (segment (start 26.62 27.75) (end 45.2125 27.75) (width 0.2) (layer "F.Cu") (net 5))
 (segment (start 21 22.13) (end 26.62 27.75) (width 0.2) (layer "F.Cu") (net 5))
 (segment (start 45.2125 27.75) (end 44.4865 28.476) (width 0.2) (layer "F.Cu") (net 5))
 (segment (start 44.4865 28.476) (end 44.4865 34.774) (width 0.2) (layer "F.Cu") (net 5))
 (segment (start 34.77375 48.68375) (end 28.62 42.53) (width 0.2) (layer "F.Cu") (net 1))
 (segment (start 28.62 42.53) (end 28.62 37.37) (width 0.2) (layer "F.Cu") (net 1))
 (segment (start 34.77375 68) (end 34.77375 48.68375) (width 0.2) (layer "F.Cu") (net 1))
 (segment (start 52.318814 48.67) (end 48.377814 52.611) (width 0.2) (layer "F.Cu") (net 9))
 (segment (start 48.377814 56.94435) (end 35.520164 69.802) (width 0.2) (layer "F.Cu") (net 9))
 (segment (start 54.1475 48.67) (end 52.318814 48.67) (width 0.2) (layer "F.Cu") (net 9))
 (segment (start 25.95275 37.49725) (end 26.08 37.37) (width 0.2) (layer "F.Cu") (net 9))
 (segment (start 54.1475 68) (end 54.1475 48.67) (width 0.2) (layer "F.Cu") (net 9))
 (segment (start 48.377814 52.611) (end 48.377814 56.94435) (width 0.2) (layer "F.Cu") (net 9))
 (segment (start 34.027336 69.802) (end 25.95275 61.727414) (width 0.2) (layer "F.Cu") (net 9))
 (segment (start 35.520164 69.802) (end 34.027336 69.802) (width 0.2) (layer "F.Cu") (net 9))
 (segment (start 25.95275 61.727414) (end 25.95275 37.49725) (width 0.2) (layer "F.Cu") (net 9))
 (segment (start 26.3 75.9) (end 23.54 73.14) (width 0.2) (layer "F.Cu") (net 13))
 (segment (start 73.5025 73.864816) (end 71.467316 75.9) (width 0.2) (layer "F.Cu") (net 13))
 (segment (start 23.54 73.14) (end 23.54 37.37) (width 0.2) (layer "F.Cu") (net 13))
 (segment (start 73.5025 68) (end 73.5025 73.864816) (width 0.2) (layer "F.Cu") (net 13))
 (segment (start 73.5025 68) (end 73.5025 48.67) (width 0.2) (layer "F.Cu") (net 13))
 (segment (start 71.467316 75.9) (end 26.3 75.9) (width 0.2) (layer "F.Cu") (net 13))
 (segment (start 100.4145 26.295008) (end 92.419492 18.3) (width 0.2) (layer "F.Cu") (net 18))
 (segment (start 92.419492 18.3) (end 31.2 18.3) (width 0.2) (layer "F.Cu") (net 18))
 (segment (start 31.2 18.3) (end 31.2 18.198) (width 0.2) (layer "F.Cu") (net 18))
 (segment (start 98.7125 32) (end 100.4145 30.298) (width 0.2) (layer "F.Cu") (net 18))
 (segment (start 100.4145 30.298) (end 100.4145 26.295008) (width 0.2) (layer "F.Cu") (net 18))
 (via (at 31.2 18.198) (size 0.6) (drill 0.3) (layers "F.Cu" "B.Cu") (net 18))
 (segment (start 31.16 18.238) (end 31.16 22.13) (width 0.2) (layer "B.Cu") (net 18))
 (segment (start 31.2 18.198) (end 31.16 18.238) (width 0.2) (layer "B.Cu") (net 18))
 (segment (start 84.2125 38.8875) (end 79.9 43.2) (width 0.2) (layer "F.Cu") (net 12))
 (segment (start 92.8125 68) (end 92.8125 40.6) (width 0.2) (layer "F.Cu") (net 12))
 (segment (start 84.2125 32) (end 84.2125 38.8875) (width 0.2) (layer "F.Cu") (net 12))
 (segment (start 92.8125 40.6) (end 84.2125 32) (width 0.2) (layer "F.Cu") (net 12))
 (via (at 79.9 43.2) (size 0.6) (drill 0.3) (layers "F.Cu" "B.Cu") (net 12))
 (segment (start 28.031 44.401) (end 21 37.37) (width 0.2) (layer "B.Cu") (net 12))
 (segment (start 79.9 43.2) (end 79.4 42.7) (width 0.2) (layer "B.Cu") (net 12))
 (segment (start 79.4 42.7) (end 55.549943 42.7) (width 0.2) (layer "B.Cu") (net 12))
 (segment (start 55.549943 42.7) (end 53.848943 44.401) (width 0.2) (layer "B.Cu") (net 12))
 (segment (start 53.848943 44.401) (end 28.031 44.401) (width 0.2) (layer "B.Cu") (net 12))
 (segment (start 28.62 21.05237) (end 30.47337 19.199) (width 0.2) (layer "F.Cu") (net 19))
 (segment (start 90.9115 19.199) (end 98.7125 27) (width 0.2) (layer "F.Cu") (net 19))
 (segment (start 30.47337 19.199) (end 90.9115 19.199) (width 0.2) (layer "F.Cu") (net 19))
 (segment (start 28.62 22.13) (end 28.62 21.05237) (width 0.2) (layer "F.Cu") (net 19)))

